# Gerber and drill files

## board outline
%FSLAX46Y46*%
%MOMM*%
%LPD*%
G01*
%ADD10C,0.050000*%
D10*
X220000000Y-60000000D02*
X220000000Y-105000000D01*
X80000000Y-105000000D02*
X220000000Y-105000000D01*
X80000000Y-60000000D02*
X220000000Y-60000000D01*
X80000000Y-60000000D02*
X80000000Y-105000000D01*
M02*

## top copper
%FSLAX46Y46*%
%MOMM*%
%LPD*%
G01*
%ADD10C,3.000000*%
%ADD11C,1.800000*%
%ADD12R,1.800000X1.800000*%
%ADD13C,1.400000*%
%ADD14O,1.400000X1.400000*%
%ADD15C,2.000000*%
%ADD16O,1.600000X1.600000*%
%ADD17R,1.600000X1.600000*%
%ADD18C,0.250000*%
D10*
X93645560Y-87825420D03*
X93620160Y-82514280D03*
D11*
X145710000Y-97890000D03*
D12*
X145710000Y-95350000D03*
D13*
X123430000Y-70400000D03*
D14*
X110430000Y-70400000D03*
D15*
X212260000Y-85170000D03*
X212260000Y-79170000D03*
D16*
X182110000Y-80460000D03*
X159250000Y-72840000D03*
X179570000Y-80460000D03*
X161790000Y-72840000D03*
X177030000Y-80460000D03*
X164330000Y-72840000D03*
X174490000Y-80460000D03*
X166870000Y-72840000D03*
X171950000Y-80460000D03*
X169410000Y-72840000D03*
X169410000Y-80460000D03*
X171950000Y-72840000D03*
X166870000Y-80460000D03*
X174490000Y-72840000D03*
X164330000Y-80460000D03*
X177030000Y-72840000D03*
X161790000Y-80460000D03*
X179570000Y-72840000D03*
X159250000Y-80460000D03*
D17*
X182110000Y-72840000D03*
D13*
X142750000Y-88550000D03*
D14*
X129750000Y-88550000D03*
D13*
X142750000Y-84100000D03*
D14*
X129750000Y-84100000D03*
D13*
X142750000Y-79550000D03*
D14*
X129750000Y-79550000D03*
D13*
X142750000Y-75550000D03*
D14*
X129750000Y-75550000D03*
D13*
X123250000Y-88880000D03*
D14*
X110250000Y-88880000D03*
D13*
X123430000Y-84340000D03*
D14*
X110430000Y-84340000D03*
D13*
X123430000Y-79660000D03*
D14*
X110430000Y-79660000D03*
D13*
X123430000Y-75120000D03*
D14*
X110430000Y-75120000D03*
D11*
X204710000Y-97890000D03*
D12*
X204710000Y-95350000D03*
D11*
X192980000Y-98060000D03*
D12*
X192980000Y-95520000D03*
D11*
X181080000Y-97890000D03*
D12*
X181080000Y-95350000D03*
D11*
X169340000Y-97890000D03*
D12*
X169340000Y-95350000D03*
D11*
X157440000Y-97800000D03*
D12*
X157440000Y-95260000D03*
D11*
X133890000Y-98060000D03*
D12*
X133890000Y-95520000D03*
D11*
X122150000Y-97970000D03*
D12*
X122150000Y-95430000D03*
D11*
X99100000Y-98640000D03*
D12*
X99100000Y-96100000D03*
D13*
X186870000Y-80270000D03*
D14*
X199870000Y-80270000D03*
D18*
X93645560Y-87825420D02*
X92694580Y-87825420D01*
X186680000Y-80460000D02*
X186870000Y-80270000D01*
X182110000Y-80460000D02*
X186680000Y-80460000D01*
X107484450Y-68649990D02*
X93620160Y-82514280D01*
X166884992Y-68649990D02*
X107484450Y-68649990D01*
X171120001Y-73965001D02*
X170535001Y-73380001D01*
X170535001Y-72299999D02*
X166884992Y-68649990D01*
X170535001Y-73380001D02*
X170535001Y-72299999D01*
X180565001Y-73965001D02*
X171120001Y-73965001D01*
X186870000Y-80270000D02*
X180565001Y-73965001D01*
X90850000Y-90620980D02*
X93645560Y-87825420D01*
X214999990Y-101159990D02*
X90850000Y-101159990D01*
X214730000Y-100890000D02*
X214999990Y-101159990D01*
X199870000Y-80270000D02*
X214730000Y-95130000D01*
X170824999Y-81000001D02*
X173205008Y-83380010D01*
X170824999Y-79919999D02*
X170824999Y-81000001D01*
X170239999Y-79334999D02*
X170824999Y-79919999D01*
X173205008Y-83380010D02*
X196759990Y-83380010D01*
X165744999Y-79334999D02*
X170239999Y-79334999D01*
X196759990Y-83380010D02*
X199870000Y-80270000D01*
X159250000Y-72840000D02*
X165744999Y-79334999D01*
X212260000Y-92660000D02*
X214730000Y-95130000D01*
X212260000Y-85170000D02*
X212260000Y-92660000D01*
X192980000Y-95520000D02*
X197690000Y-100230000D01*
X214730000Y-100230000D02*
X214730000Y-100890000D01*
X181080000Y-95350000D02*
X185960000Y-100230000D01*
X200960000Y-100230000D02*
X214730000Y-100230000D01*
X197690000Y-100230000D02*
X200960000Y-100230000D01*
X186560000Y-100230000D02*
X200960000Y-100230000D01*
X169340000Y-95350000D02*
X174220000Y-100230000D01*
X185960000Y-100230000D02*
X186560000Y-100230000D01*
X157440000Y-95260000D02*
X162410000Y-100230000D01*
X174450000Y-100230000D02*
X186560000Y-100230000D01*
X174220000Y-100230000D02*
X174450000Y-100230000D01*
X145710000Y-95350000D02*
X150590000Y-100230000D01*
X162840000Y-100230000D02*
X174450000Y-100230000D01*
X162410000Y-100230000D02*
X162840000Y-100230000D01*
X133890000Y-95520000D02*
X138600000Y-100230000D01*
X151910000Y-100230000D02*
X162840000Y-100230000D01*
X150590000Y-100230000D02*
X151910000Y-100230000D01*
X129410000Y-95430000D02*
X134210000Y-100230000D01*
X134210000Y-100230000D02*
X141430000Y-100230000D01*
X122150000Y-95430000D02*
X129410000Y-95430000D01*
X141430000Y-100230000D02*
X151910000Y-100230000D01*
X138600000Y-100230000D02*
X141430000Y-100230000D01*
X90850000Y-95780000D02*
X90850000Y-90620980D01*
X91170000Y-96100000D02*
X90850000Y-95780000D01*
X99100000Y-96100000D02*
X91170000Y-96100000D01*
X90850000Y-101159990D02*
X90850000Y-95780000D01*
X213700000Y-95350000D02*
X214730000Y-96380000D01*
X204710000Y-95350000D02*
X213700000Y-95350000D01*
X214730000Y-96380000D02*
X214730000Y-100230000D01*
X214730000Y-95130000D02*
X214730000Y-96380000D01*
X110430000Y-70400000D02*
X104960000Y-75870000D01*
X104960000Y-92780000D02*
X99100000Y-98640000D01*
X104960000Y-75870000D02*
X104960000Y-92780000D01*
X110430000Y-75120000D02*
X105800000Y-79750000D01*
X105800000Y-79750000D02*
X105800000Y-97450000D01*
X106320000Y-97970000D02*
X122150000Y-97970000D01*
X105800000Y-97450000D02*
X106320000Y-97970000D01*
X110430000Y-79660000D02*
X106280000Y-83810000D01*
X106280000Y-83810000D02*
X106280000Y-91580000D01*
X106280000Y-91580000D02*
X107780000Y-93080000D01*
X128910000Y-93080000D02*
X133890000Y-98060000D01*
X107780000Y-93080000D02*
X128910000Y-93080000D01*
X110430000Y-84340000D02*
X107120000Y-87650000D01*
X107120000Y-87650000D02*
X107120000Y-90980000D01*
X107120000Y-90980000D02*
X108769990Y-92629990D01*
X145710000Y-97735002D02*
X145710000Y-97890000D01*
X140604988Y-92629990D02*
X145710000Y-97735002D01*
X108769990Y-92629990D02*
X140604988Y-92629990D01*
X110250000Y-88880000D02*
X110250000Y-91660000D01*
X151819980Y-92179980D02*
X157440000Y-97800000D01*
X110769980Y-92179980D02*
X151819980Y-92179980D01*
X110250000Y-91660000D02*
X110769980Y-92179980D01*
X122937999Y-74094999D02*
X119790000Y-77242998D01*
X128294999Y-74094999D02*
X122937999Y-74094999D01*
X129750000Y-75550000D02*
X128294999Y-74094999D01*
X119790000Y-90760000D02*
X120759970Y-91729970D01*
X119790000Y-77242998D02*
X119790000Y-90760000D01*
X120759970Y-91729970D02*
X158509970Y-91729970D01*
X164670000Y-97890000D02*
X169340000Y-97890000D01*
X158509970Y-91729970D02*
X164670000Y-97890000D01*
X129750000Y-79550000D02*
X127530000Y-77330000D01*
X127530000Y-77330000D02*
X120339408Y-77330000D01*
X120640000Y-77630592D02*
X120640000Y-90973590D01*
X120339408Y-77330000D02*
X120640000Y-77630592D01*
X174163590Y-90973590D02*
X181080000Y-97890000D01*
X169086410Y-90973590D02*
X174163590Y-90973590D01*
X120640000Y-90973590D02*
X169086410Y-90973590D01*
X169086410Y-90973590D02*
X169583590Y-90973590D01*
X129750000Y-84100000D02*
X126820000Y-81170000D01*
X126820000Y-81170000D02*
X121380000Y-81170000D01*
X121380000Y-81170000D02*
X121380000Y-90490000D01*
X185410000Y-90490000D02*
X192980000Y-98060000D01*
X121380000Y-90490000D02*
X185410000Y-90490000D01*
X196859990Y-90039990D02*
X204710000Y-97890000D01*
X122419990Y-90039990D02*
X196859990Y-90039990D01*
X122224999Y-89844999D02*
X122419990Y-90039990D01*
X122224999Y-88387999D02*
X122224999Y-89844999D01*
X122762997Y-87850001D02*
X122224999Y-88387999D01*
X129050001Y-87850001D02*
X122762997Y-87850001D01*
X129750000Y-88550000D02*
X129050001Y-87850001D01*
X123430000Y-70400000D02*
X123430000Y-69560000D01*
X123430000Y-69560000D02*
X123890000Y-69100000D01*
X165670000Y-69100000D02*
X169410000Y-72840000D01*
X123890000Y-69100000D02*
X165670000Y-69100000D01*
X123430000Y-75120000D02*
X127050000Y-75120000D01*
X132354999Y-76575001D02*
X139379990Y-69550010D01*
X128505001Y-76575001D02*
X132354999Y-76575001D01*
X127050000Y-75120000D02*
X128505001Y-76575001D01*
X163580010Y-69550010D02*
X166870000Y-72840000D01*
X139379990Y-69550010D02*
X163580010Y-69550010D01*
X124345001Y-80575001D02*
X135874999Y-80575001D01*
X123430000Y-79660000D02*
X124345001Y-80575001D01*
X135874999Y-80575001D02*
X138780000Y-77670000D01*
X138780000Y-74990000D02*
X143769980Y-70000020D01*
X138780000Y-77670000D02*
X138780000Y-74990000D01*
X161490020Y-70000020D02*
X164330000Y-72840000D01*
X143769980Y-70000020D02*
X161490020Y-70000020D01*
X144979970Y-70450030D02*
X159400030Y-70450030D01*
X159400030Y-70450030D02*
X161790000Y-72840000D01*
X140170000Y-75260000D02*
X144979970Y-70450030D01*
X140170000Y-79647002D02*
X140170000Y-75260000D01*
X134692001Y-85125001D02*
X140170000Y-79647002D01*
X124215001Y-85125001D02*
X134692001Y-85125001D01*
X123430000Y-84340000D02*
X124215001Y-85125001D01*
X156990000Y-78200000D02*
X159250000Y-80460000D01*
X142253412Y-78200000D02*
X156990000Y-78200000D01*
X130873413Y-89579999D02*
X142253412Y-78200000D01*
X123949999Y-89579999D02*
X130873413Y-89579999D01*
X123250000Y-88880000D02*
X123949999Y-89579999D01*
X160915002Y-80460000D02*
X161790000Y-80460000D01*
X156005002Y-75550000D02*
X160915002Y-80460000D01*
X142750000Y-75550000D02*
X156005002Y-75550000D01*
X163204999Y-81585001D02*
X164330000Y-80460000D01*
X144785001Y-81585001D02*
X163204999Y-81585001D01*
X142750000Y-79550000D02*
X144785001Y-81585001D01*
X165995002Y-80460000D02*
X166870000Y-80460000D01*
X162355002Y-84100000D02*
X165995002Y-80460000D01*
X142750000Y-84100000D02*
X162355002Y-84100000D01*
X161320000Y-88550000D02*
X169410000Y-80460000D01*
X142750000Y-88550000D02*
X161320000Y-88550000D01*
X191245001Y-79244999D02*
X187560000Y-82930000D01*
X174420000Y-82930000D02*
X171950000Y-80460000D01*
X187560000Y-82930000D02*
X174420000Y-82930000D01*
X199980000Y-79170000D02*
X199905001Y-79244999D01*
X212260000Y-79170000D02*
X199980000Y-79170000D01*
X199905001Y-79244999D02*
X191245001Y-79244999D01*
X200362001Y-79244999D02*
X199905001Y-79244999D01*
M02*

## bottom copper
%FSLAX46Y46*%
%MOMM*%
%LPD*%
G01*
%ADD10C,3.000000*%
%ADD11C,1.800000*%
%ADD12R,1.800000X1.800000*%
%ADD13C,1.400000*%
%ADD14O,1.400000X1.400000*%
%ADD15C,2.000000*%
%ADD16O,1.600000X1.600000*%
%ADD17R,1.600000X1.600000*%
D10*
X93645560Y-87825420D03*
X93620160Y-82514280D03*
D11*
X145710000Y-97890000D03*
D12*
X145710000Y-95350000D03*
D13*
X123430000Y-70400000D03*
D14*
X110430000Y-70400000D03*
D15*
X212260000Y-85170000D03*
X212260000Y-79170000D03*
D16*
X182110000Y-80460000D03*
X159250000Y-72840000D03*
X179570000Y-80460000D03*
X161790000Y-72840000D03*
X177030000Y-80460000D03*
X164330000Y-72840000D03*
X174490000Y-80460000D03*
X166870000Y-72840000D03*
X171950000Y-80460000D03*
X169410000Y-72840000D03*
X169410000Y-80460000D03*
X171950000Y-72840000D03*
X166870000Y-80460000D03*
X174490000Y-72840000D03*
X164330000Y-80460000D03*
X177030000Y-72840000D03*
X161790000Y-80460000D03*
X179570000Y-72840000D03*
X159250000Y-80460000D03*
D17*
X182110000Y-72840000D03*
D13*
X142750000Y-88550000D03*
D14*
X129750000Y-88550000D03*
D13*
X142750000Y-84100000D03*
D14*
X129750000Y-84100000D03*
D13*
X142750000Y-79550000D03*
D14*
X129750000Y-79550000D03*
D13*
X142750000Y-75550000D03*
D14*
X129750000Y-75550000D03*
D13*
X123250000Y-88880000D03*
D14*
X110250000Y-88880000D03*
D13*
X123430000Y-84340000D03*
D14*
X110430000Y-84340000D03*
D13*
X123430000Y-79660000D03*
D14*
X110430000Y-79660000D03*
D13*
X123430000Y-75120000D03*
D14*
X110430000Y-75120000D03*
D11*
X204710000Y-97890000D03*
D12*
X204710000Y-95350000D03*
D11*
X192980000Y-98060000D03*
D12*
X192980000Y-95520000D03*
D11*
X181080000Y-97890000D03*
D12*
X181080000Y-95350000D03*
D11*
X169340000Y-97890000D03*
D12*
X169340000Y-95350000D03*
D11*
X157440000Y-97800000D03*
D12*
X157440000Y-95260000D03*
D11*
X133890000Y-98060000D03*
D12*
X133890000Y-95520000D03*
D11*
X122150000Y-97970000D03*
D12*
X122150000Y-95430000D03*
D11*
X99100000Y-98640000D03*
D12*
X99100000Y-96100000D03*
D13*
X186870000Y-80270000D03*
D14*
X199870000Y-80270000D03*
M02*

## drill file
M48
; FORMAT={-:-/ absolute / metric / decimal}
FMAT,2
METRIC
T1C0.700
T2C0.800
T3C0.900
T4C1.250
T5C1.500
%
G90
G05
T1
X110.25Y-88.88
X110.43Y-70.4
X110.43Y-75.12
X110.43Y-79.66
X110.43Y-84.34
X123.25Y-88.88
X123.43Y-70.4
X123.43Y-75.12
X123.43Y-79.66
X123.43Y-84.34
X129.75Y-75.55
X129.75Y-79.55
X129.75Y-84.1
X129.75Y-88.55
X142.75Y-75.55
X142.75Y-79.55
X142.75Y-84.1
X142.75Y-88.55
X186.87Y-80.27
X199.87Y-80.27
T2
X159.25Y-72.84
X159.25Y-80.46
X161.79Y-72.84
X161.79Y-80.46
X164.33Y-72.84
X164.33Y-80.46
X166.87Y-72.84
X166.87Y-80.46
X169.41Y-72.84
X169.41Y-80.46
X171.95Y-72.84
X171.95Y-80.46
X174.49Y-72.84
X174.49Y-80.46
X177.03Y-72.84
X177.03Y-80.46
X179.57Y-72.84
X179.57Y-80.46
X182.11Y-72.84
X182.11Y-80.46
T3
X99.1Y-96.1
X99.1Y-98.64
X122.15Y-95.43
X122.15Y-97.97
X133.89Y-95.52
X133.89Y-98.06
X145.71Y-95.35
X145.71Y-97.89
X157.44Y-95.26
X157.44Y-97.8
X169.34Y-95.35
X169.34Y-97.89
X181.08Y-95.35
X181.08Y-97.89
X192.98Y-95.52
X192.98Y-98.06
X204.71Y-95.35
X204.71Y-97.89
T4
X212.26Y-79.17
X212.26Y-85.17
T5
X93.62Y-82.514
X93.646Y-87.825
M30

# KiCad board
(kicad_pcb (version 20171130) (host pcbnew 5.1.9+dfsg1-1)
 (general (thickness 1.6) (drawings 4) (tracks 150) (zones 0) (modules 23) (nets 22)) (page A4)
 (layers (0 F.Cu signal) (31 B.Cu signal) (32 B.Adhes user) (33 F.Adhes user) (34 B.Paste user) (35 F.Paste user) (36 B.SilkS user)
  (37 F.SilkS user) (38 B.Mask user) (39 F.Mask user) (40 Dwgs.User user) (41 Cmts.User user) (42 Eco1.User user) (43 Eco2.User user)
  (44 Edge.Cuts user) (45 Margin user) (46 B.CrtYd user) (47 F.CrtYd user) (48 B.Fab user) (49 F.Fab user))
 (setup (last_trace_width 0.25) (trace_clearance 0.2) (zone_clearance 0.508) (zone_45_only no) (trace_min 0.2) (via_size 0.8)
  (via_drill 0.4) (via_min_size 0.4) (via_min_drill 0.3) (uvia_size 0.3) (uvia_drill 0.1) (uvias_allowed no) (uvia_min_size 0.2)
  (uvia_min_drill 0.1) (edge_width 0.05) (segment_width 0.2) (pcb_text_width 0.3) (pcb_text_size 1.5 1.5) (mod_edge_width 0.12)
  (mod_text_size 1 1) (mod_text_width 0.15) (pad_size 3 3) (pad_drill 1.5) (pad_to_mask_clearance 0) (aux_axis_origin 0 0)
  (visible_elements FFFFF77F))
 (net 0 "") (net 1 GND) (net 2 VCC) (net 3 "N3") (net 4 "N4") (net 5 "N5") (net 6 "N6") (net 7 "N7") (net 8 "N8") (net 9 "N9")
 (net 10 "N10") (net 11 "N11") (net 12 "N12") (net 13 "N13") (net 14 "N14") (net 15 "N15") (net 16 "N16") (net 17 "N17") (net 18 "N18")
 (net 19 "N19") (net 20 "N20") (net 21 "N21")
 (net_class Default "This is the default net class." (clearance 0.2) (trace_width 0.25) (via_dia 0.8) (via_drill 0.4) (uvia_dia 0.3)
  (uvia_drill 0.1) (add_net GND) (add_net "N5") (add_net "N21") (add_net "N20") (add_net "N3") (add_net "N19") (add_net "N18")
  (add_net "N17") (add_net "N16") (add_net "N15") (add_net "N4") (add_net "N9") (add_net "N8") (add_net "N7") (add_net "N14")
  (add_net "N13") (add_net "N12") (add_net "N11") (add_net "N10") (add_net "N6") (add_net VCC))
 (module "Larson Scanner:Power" (layer F.Cu) (at 93.61 85.1)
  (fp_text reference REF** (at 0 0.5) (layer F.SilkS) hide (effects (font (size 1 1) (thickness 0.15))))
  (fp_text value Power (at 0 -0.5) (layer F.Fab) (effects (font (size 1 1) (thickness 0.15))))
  (pad 2 thru_hole circle (at 0.03556 2.72542) (size 3 3) (drill 1.5) (layers *.Cu *.Mask) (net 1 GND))
  (pad 1 thru_hole circle (at 0.01016 -2.58572) (size 3 3) (drill 1.5) (layers *.Cu *.Mask) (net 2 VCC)))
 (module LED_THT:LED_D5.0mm (layer F.Cu) (at 145.71 95.35 270)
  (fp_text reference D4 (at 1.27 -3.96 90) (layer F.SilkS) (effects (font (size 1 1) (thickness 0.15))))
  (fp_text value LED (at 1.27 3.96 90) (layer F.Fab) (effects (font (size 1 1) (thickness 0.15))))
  (pad 2 thru_hole circle (at 2.54 0 270) (size 1.8 1.8) (drill 0.9) (layers *.Cu *.Mask) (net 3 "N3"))
  (pad 1 thru_hole rect (at 0 0 270) (size 1.8 1.8) (drill 0.9) (layers *.Cu *.Mask) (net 1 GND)))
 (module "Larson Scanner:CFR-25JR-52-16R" (layer F.Cu) (at 116.93 70.4 180)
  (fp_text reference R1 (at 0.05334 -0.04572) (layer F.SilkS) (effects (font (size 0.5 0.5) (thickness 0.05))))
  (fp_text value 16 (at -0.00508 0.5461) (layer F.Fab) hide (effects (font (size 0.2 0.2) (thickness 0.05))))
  (pad 1 thru_hole circle (at -6.5 0 180) (size 1.4 1.4) (drill 0.7) (layers *.Cu *.Mask) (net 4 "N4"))
  (pad 2 thru_hole oval (at 6.5 0 180) (size 1.4 1.4) (drill 0.7) (layers *.Cu *.Mask) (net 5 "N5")))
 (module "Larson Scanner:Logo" (layer F.Cu) (at 98.32 68.52)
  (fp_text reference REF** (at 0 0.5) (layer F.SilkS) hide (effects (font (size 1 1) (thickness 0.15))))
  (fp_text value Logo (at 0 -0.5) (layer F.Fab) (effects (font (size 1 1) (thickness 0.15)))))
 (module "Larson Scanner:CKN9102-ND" (layer F.Cu) (at 212.26 82.17)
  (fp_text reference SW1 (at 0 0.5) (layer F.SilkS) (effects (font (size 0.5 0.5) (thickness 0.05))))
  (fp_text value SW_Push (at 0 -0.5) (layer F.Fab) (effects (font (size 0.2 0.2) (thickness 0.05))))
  (pad 2 thru_hole circle (at 0 3 180) (size 2 2) (drill 1.25) (layers *.Cu *.Mask) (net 1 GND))
  (pad 1 thru_hole circle (at 0 -3 180) (size 2 2) (drill 1.25) (layers *.Cu *.Mask) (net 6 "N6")))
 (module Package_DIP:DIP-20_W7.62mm (layer F.Cu) (at 182.11 72.84 270)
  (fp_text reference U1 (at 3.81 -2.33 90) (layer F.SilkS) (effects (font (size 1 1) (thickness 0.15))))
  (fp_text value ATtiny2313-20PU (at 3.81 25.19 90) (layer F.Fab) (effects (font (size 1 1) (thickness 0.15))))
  (pad 20 thru_hole oval (at 7.62 0 270) (size 1.6 1.6) (drill 0.8) (layers *.Cu *.Mask) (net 2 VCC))
  (pad 10 thru_hole oval (at 0 22.86 270) (size 1.6 1.6) (drill 0.8) (layers *.Cu *.Mask) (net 1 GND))
  (pad 19 thru_hole oval (at 7.62 2.54 270) (size 1.6 1.6) (drill 0.8) (layers *.Cu *.Mask))
  (pad 9 thru_hole oval (at 0 20.32 270) (size 1.6 1.6) (drill 0.8) (layers *.Cu *.Mask) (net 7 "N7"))
  (pad 18 thru_hole oval (at 7.62 5.08 270) (size 1.6 1.6) (drill 0.8) (layers *.Cu *.Mask))
  (pad 8 thru_hole oval (at 0 17.78 270) (size 1.6 1.6) (drill 0.8) (layers *.Cu *.Mask) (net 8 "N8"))
  (pad 17 thru_hole oval (at 7.62 7.62 270) (size 1.6 1.6) (drill 0.8) (layers *.Cu *.Mask))
  (pad 7 thru_hole oval (at 0 15.24 270) (size 1.6 1.6) (drill 0.8) (layers *.Cu *.Mask) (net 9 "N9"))
  (pad 16 thru_hole oval (at 7.62 10.16 270) (size 1.6 1.6) (drill 0.8) (layers *.Cu *.Mask) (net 6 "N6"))
  (pad 6 thru_hole oval (at 0 12.7 270) (size 1.6 1.6) (drill 0.8) (layers *.Cu *.Mask) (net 4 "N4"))
  (pad 15 thru_hole oval (at 7.62 12.7 270) (size 1.6 1.6) (drill 0.8) (layers *.Cu *.Mask) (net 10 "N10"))
  (pad 5 thru_hole oval (at 0 10.16 270) (size 1.6 1.6) (drill 0.8) (layers *.Cu *.Mask))
  (pad 14 thru_hole oval (at 7.62 15.24 270) (size 1.6 1.6) (drill 0.8) (layers *.Cu *.Mask) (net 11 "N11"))
  (pad 4 thru_hole oval (at 0 7.62 270) (size 1.6 1.6) (drill 0.8) (layers *.Cu *.Mask))
  (pad 13 thru_hole oval (at 7.62 17.78 270) (size 1.6 1.6) (drill 0.8) (layers *.Cu *.Mask) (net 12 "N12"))
  (pad 3 thru_hole oval (at 0 5.08 270) (size 1.6 1.6) (drill 0.8) (layers *.Cu *.Mask))
  (pad 12 thru_hole oval (at 7.62 20.32 270) (size 1.6 1.6) (drill 0.8) (layers *.Cu *.Mask) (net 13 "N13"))
  (pad 2 thru_hole oval (at 0 2.54 270) (size 1.6 1.6) (drill 0.8) (layers *.Cu *.Mask))
  (pad 11 thru_hole oval (at 7.62 22.86 270) (size 1.6 1.6) (drill 0.8) (layers *.Cu *.Mask) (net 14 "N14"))
  (pad 1 thru_hole rect (at 0 0 270) (size 1.6 1.6) (drill 0.8) (layers *.Cu *.Mask)))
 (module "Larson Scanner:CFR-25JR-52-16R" (layer F.Cu) (at 136.25 88.55 180)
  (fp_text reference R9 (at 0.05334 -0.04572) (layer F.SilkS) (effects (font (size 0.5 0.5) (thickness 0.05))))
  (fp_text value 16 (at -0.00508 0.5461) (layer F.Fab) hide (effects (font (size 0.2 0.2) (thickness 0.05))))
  (pad 1 thru_hole circle (at -6.5 0 180) (size 1.4 1.4) (drill 0.7) (layers *.Cu *.Mask) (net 10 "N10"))
  (pad 2 thru_hole oval (at 6.5 0 180) (size 1.4 1.4) (drill 0.7) (layers *.Cu *.Mask) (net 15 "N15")))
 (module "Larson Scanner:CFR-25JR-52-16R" (layer F.Cu) (at 136.25 84.1 180)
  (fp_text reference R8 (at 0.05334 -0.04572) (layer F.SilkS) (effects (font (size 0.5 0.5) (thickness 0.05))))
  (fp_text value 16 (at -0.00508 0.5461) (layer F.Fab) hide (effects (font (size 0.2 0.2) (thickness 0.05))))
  (pad 1 thru_hole circle (at -6.5 0 180) (size 1.4 1.4) (drill 0.7) (layers *.Cu *.Mask) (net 11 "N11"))
  (pad 2 thru_hole oval (at 6.5 0 180) (size 1.4 1.4) (drill 0.7) (layers *.Cu *.Mask) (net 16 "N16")))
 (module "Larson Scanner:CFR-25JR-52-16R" (layer F.Cu) (at 136.25 79.55 180)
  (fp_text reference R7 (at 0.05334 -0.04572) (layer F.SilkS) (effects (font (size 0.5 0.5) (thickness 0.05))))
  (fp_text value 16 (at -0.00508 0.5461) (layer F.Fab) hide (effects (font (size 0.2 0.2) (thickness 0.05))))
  (pad 1 thru_hole circle (at -6.5 0 180) (size 1.4 1.4) (drill 0.7) (layers *.Cu *.Mask) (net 12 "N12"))
  (pad 2 thru_hole oval (at 6.5 0 180) (size 1.4 1.4) (drill 0.7) (layers *.Cu *.Mask) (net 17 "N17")))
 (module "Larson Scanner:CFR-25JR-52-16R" (layer F.Cu) (at 136.25 75.55 180)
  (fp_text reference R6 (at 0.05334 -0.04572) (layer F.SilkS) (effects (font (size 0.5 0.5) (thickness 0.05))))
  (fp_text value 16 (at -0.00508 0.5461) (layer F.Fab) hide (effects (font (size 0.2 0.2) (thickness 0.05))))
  (pad 1 thru_hole circle (at -6.5 0 180) (size 1.4 1.4) (drill 0.7) (layers *.Cu *.Mask) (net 13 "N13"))
  (pad 2 thru_hole oval (at 6.5 0 180) (size 1.4 1.4) (drill 0.7) (layers *.Cu *.Mask) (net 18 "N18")))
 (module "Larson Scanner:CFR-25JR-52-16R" (layer F.Cu) (at 116.75 88.88 180)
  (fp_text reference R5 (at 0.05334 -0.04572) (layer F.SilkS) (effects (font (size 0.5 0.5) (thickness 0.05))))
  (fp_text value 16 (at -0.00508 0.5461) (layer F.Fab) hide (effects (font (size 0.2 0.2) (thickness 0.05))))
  (pad 1 thru_hole circle (at -6.5 0 180) (size 1.4 1.4) (drill 0.7) (layers *.Cu *.Mask) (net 14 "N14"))
  (pad 2 thru_hole oval (at 6.5 0 180) (size 1.4 1.4) (drill 0.7) (layers *.Cu *.Mask) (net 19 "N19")))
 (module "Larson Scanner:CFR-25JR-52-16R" (layer F.Cu) (at 116.93 84.34 180)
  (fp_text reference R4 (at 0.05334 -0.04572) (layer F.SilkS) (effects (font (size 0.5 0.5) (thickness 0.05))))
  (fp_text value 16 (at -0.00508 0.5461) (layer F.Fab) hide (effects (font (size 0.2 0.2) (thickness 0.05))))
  (pad 1 thru_hole circle (at -6.5 0 180) (size 1.4 1.4) (drill 0.7) (layers *.Cu *.Mask) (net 7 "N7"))
  (pad 2 thru_hole oval (at 6.5 0 180) (size 1.4 1.4) (drill 0.7) (layers *.Cu *.Mask) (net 3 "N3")))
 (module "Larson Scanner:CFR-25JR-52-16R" (layer F.Cu) (at 116.93 79.66 180)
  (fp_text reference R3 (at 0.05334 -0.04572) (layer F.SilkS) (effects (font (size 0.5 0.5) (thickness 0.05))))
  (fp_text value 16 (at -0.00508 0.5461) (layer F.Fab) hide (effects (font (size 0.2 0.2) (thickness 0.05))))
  (pad 1 thru_hole circle (at -6.5 0 180) (size 1.4 1.4) (drill 0.7) (layers *.Cu *.Mask) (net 8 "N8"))
  (pad 2 thru_hole oval (at 6.5 0 180) (size 1.4 1.4) (drill 0.7) (layers *.Cu *.Mask) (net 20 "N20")))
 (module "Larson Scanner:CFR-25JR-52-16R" (layer F.Cu) (at 116.93 75.12 180)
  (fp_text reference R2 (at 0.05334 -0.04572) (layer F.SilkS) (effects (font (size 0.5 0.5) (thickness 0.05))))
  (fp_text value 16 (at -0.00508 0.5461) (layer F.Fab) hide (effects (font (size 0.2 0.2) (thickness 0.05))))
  (pad 1 thru_hole circle (at -6.5 0 180) (size 1.4 1.4) (drill 0.7) (layers *.Cu *.Mask) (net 9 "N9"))
  (pad 2 thru_hole oval (at 6.5 0 180) (size 1.4 1.4) (drill 0.7) (layers *.Cu *.Mask) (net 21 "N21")))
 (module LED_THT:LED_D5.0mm (layer F.Cu) (at 204.71 95.35 270)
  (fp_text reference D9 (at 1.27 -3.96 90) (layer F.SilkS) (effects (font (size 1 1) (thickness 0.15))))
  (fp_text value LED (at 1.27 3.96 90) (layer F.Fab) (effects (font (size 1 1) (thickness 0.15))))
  (pad 2 thru_hole circle (at 2.54 0 270) (size 1.8 1.8) (drill 0.9) (layers *.Cu *.Mask) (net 15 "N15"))
  (pad 1 thru_hole rect (at 0 0 270) (size 1.8 1.8) (drill 0.9) (layers *.Cu *.Mask) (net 1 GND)))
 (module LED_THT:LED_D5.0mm (layer F.Cu) (at 192.98 95.52 270)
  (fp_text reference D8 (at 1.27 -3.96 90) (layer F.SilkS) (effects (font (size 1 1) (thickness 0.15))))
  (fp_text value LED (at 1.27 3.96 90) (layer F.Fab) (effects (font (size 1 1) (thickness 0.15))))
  (pad 2 thru_hole circle (at 2.54 0 270) (size 1.8 1.8) (drill 0.9) (layers *.Cu *.Mask) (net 16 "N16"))
  (pad 1 thru_hole rect (at 0 0 270) (size 1.8 1.8) (drill 0.9) (layers *.Cu *.Mask) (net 1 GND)))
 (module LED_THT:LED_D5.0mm (layer F.Cu) (at 181.08 95.35 270)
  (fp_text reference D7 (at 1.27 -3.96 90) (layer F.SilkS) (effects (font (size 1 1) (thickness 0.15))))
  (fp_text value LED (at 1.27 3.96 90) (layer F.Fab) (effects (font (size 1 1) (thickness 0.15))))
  (pad 2 thru_hole circle (at 2.54 0 270) (size 1.8 1.8) (drill 0.9) (layers *.Cu *.Mask) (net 17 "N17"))
  (pad 1 thru_hole rect (at 0 0 270) (size 1.8 1.8) (drill 0.9) (layers *.Cu *.Mask) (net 1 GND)))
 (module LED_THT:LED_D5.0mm (layer F.Cu) (at 169.34 95.35 270)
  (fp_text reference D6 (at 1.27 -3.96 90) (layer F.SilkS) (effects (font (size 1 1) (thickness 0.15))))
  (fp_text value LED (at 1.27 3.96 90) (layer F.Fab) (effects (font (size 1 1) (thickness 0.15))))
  (pad 2 thru_hole circle (at 2.54 0 270) (size 1.8 1.8) (drill 0.9) (layers *.Cu *.Mask) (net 18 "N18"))
  (pad 1 thru_hole rect (at 0 0 270) (size 1.8 1.8) (drill 0.9) (layers *.Cu *.Mask) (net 1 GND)))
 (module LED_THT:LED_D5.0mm (layer F.Cu) (at 157.44 95.26 270)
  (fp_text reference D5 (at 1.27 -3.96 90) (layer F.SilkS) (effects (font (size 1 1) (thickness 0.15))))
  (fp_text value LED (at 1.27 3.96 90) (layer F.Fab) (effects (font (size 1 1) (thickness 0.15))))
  (pad 2 thru_hole circle (at 2.54 0 270) (size 1.8 1.8) (drill 0.9) (layers *.Cu *.Mask) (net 19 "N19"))
  (pad 1 thru_hole rect (at 0 0 270) (size 1.8 1.8) (drill 0.9) (layers *.Cu *.Mask) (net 1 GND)))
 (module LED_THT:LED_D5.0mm (layer F.Cu) (at 133.89 95.52 270)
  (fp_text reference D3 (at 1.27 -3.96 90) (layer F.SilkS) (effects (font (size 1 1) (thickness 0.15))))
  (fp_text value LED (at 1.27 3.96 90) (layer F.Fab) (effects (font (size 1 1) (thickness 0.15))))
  (pad 2 thru_hole circle (at 2.54 0 270) (size 1.8 1.8) (drill 0.9) (layers *.Cu *.Mask) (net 20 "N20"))
  (pad 1 thru_hole rect (at 0 0 270) (size 1.8 1.8) (drill 0.9) (layers *.Cu *.Mask) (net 1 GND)))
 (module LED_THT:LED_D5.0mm (layer F.Cu) (at 122.15 95.43 270)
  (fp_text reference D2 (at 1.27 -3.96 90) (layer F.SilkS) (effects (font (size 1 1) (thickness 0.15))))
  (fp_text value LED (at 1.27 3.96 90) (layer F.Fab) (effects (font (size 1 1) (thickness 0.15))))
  (pad 2 thru_hole circle (at 2.54 0 270) (size 1.8 1.8) (drill 0.9) (layers *.Cu *.Mask) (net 21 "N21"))
  (pad 1 thru_hole rect (at 0 0 270) (size 1.8 1.8) (drill 0.9) (layers *.Cu *.Mask) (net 1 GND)))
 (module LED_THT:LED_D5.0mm (layer F.Cu) (at 99.1 96.1 270)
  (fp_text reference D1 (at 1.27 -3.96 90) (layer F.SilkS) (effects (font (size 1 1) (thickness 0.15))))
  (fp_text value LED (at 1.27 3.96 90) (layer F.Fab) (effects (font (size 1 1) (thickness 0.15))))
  (pad 2 thru_hole circle (at 2.54 0 270) (size 1.8 1.8) (drill 0.9) (layers *.Cu *.Mask) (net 5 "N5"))
  (pad 1 thru_hole rect (at 0 0 270) (size 1.8 1.8) (drill 0.9) (layers *.Cu *.Mask) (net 1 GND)))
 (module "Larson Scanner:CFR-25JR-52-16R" (layer F.Cu) (at 193.37 80.27)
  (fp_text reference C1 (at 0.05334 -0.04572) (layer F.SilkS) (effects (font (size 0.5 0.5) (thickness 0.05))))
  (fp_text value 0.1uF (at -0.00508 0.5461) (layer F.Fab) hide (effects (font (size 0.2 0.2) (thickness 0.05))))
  (pad 1 thru_hole circle (at -6.5 0) (size 1.4 1.4) (drill 0.7) (layers *.Cu *.Mask) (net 2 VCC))
  (pad 2 thru_hole oval (at 6.5 0) (size 1.4 1.4) (drill 0.7) (layers *.Cu *.Mask) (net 1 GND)))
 (gr_line (start 220 60) (end 220 105) (layer Edge.Cuts) (width 0.05))
 (gr_line (start 80 105) (end 220 105) (layer Edge.Cuts) (width 0.05))
 (gr_line (start 80 60) (end 220 60) (layer Edge.Cuts) (width 0.05))
 (gr_line (start 80 60) (end 80 105) (layer Edge.Cuts) (width 0.05))
 (segment (start 93.64556 87.82542) (end 92.69458 87.82542) (width 0.25) (layer F.Cu) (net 1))
 (segment (start 186.68 80.46) (end 186.87 80.27) (width 0.25) (layer F.Cu) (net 2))
 (segment (start 182.11 80.46) (end 186.68 80.46) (width 0.25) (layer F.Cu) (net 2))
 (segment (start 107.48445 68.64999) (end 93.62016 82.51428) (width 0.25) (layer F.Cu) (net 2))
 (segment (start 166.884992 68.64999) (end 107.48445 68.64999) (width 0.25) (layer F.Cu) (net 2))
 (segment (start 171.120001 73.965001) (end 170.535001 73.380001) (width 0.25) (layer F.Cu) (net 2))
 (segment (start 170.535001 72.299999) (end 166.884992 68.64999) (width 0.25) (layer F.Cu) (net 2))
 (segment (start 170.535001 73.380001) (end 170.535001 72.299999) (width 0.25) (layer F.Cu) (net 2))
 (segment (start 180.565001 73.965001) (end 171.120001 73.965001) (width 0.25) (layer F.Cu) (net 2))
 (segment (start 186.87 80.27) (end 180.565001 73.965001) (width 0.25) (layer F.Cu) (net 2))
 (segment (start 90.85 90.62098) (end 93.64556 87.82542) (width 0.25) (layer F.Cu) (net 1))
 (segment (start 214.99999 101.15999) (end 90.85 101.15999) (width 0.25) (layer F.Cu) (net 1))
 (segment (start 214.73 100.89) (end 214.99999 101.15999) (width 0.25) (layer F.Cu) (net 1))
 (segment (start 199.87 80.27) (end 214.73 95.13) (width 0.25) (layer F.Cu) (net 1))
 (segment (start 170.824999 81.000001) (end 173.205008 83.38001) (width 0.25) (layer F.Cu) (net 1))
 (segment (start 170.824999 79.919999) (end 170.824999 81.000001) (width 0.25) (layer F.Cu) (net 1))
 (segment (start 170.239999 79.334999) (end 170.824999 79.919999) (width 0.25) (layer F.Cu) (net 1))
 (segment (start 173.205008 83.38001) (end 196.75999 83.38001) (width 0.25) (layer F.Cu) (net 1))
 (segment (start 165.744999 79.334999) (end 170.239999 79.334999) (width 0.25) (layer F.Cu) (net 1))
 (segment (start 196.75999 83.38001) (end 199.87 80.27) (width 0.25) (layer F.Cu) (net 1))
 (segment (start 159.25 72.84) (end 165.744999 79.334999) (width 0.25) (layer F.Cu) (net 1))
 (segment (start 212.26 92.66) (end 214.73 95.13) (width 0.25) (layer F.Cu) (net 1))
 (segment (start 212.26 85.17) (end 212.26 92.66) (width 0.25) (layer F.Cu) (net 1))
 (segment (start 192.98 95.52) (end 197.69 100.23) (width 0.25) (layer F.Cu) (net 1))
 (segment (start 214.73 100.23) (end 214.73 100.89) (width 0.25) (layer F.Cu) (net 1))
 (segment (start 181.08 95.35) (end 185.96 100.23) (width 0.25) (layer F.Cu) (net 1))
 (segment (start 200.96 100.23) (end 214.73 100.23) (width 0.25) (layer F.Cu) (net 1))
 (segment (start 197.69 100.23) (end 200.96 100.23) (width 0.25) (layer F.Cu) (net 1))
 (segment (start 186.56 100.23) (end 200.96 100.23) (width 0.25) (layer F.Cu) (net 1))
 (segment (start 169.34 95.35) (end 174.22 100.23) (width 0.25) (layer F.Cu) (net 1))
 (segment (start 185.96 100.23) (end 186.56 100.23) (width 0.25) (layer F.Cu) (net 1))
 (segment (start 157.44 95.26) (end 162.41 100.23) (width 0.25) (layer F.Cu) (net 1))
 (segment (start 174.45 100.23) (end 186.56 100.23) (width 0.25) (layer F.Cu) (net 1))
 (segment (start 174.22 100.23) (end 174.45 100.23) (width 0.25) (layer F.Cu) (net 1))
 (segment (start 145.71 95.35) (end 150.59 100.23) (width 0.25) (layer F.Cu) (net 1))
 (segment (start 162.84 100.23) (end 174.45 100.23) (width 0.25) (layer F.Cu) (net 1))
 (segment (start 162.41 100.23) (end 162.84 100.23) (width 0.25) (layer F.Cu) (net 1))
 (segment (start 133.89 95.52) (end 138.6 100.23) (width 0.25) (layer F.Cu) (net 1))
 (segment (start 151.91 100.23) (end 162.84 100.23) (width 0.25) (layer F.Cu) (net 1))
 (segment (start 150.59 100.23) (end 151.91 100.23) (width 0.25) (layer F.Cu) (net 1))
 (segment (start 129.41 95.43) (end 134.21 100.23) (width 0.25) (layer F.Cu) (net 1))
 (segment (start 134.21 100.23) (end 141.43 100.23) (width 0.25) (layer F.Cu) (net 1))
 (segment (start 122.15 95.43) (end 129.41 95.43) (width 0.25) (layer F.Cu) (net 1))
 (segment (start 141.43 100.23) (end 151.91 100.23) (width 0.25) (layer F.Cu) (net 1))
 (segment (start 138.6 100.23) (end 141.43 100.23) (width 0.25) (layer F.Cu) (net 1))
 (segment (start 90.85 95.78) (end 90.85 90.62098) (width 0.25) (layer F.Cu) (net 1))
 (segment (start 91.17 96.1) (end 90.85 95.78) (width 0.25) (layer F.Cu) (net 1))
 (segment (start 99.1 96.1) (end 91.17 96.1) (width 0.25) (layer F.Cu) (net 1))
 (segment (start 90.85 101.15999) (end 90.85 95.78) (width 0.25) (layer F.Cu) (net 1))
 (segment (start 213.7 95.35) (end 214.73 96.38) (width 0.25) (layer F.Cu) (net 1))
 (segment (start 204.71 95.35) (end 213.7 95.35) (width 0.25) (layer F.Cu) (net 1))
 (segment (start 214.73 96.38) (end 214.73 100.23) (width 0.25) (layer F.Cu) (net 1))
 (segment (start 214.73 95.13) (end 214.73 96.38) (width 0.25) (layer F.Cu) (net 1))
 (segment (start 110.43 70.4) (end 104.96 75.87) (width 0.25) (layer F.Cu) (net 5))
 (segment (start 104.96 92.78) (end 99.1 98.64) (width 0.25) (layer F.Cu) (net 5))
 (segment (start 104.96 75.87) (end 104.96 92.78) (width 0.25) (layer F.Cu) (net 5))
 (segment (start 110.43 75.12) (end 105.8 79.75) (width 0.25) (layer F.Cu) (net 21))
 (segment (start 105.8 79.75) (end 105.8 97.45) (width 0.25) (layer F.Cu) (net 21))
 (segment (start 106.32 97.97) (end 122.15 97.97) (width 0.25) (layer F.Cu) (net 21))
 (segment (start 105.8 97.45) (end 106.32 97.97) (width 0.25) (layer F.Cu) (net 21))
 (segment (start 110.43 79.66) (end 106.28 83.81) (width 0.25) (layer F.Cu) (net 20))
 (segment (start 106.28 83.81) (end 106.28 91.58) (width 0.25) (layer F.Cu) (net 20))
 (segment (start 106.28 91.58) (end 107.78 93.08) (width 0.25) (layer F.Cu) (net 20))
 (segment (start 128.91 93.08) (end 133.89 98.06) (width 0.25) (layer F.Cu) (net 20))
 (segment (start 107.78 93.08) (end 128.91 93.08) (width 0.25) (layer F.Cu) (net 20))
 (segment (start 110.43 84.34) (end 107.12 87.65) (width 0.25) (layer F.Cu) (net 3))
 (segment (start 107.12 87.65) (end 107.12 90.98) (width 0.25) (layer F.Cu) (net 3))
 (segment (start 107.12 90.98) (end 108.76999 92.62999) (width 0.25) (layer F.Cu) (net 3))
 (segment (start 145.71 97.735002) (end 145.71 97.89) (width 0.25) (layer F.Cu) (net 3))
 (segment (start 140.604988 92.62999) (end 145.71 97.735002) (width 0.25) (layer F.Cu) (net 3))
 (segment (start 108.76999 92.62999) (end 140.604988 92.62999) (width 0.25) (layer F.Cu) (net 3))
 (segment (start 110.25 88.88) (end 110.25 91.66) (width 0.25) (layer F.Cu) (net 19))
 (segment (start 151.81998 92.17998) (end 157.44 97.8) (width 0.25) (layer F.Cu) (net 19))
 (segment (start 110.76998 92.17998) (end 151.81998 92.17998) (width 0.25) (layer F.Cu) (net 19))
 (segment (start 110.25 91.66) (end 110.76998 92.17998) (width 0.25) (layer F.Cu) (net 19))
 (segment (start 122.937999 74.094999) (end 119.79 77.242998) (width 0.25) (layer F.Cu) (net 18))
 (segment (start 128.294999 74.094999) (end 122.937999 74.094999) (width 0.25) (layer F.Cu) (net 18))
 (segment (start 129.75 75.55) (end 128.294999 74.094999) (width 0.25) (layer F.Cu) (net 18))
 (segment (start 119.79 90.76) (end 120.75997 91.72997) (width 0.25) (layer F.Cu) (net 18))
 (segment (start 119.79 77.242998) (end 119.79 90.76) (width 0.25) (layer F.Cu) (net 18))
 (segment (start 120.75997 91.72997) (end 158.50997 91.72997) (width 0.25) (layer F.Cu) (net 18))
 (segment (start 164.67 97.89) (end 169.34 97.89) (width 0.25) (layer F.Cu) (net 18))
 (segment (start 158.50997 91.72997) (end 164.67 97.89) (width 0.25) (layer F.Cu) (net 18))
 (segment (start 129.75 79.55) (end 127.53 77.33) (width 0.25) (layer F.Cu) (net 17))
 (segment (start 127.53 77.33) (end 120.339408 77.33) (width 0.25) (layer F.Cu) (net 17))
 (segment (start 120.64 77.630592) (end 120.64 90.97359) (width 0.25) (layer F.Cu) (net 17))
 (segment (start 120.339408 77.33) (end 120.64 77.630592) (width 0.25) (layer F.Cu) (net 17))
 (segment (start 174.16359 90.97359) (end 181.08 97.89) (width 0.25) (layer F.Cu) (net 17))
 (segment (start 169.08641 90.97359) (end 174.16359 90.97359) (width 0.25) (layer F.Cu) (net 17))
 (segment (start 120.64 90.97359) (end 169.08641 90.97359) (width 0.25) (layer F.Cu) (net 17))
 (segment (start 169.08641 90.97359) (end 169.58359 90.97359) (width 0.25) (layer F.Cu) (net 17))
 (segment (start 129.75 84.1) (end 126.82 81.17) (width 0.25) (layer F.Cu) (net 16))
 (segment (start 126.82 81.17) (end 121.38 81.17) (width 0.25) (layer F.Cu) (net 16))
 (segment (start 121.38 81.17) (end 121.38 90.49) (width 0.25) (layer F.Cu) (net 16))
 (segment (start 185.41 90.49) (end 192.98 98.06) (width 0.25) (layer F.Cu) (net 16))
 (segment (start 121.38 90.49) (end 185.41 90.49) (width 0.25) (layer F.Cu) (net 16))
 (segment (start 196.85999 90.03999) (end 204.71 97.89) (width 0.25) (layer F.Cu) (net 15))
 (segment (start 122.41999 90.03999) (end 196.85999 90.03999) (width 0.25) (layer F.Cu) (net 15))
 (segment (start 122.224999 89.844999) (end 122.41999 90.03999) (width 0.25) (layer F.Cu) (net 15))
 (segment (start 122.224999 88.387999) (end 122.224999 89.844999) (width 0.25) (layer F.Cu) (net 15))
 (segment (start 122.762997 87.850001) (end 122.224999 88.387999) (width 0.25) (layer F.Cu) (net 15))
 (segment (start 129.050001 87.850001) (end 122.762997 87.850001) (width 0.25) (layer F.Cu) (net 15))
 (segment (start 129.75 88.55) (end 129.050001 87.850001) (width 0.25) (layer F.Cu) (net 15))
 (segment (start 123.43 70.4) (end 123.43 69.56) (width 0.25) (layer F.Cu) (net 4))
 (segment (start 123.43 69.56) (end 123.89 69.1) (width 0.25) (layer F.Cu) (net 4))
 (segment (start 165.67 69.1) (end 169.41 72.84) (width 0.25) (layer F.Cu) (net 4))
 (segment (start 123.89 69.1) (end 165.67 69.1) (width 0.25) (layer F.Cu) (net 4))
 (segment (start 123.43 75.12) (end 127.05 75.12) (width 0.25) (layer F.Cu) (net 9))
 (segment (start 132.354999 76.575001) (end 139.37999 69.55001) (width 0.25) (layer F.Cu) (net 9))
 (segment (start 128.505001 76.575001) (end 132.354999 76.575001) (width 0.25) (layer F.Cu) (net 9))
 (segment (start 127.05 75.12) (end 128.505001 76.575001) (width 0.25) (layer F.Cu) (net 9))
 (segment (start 163.58001 69.55001) (end 166.87 72.84) (width 0.25) (layer F.Cu) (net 9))
 (segment (start 139.37999 69.55001) (end 163.58001 69.55001) (width 0.25) (layer F.Cu) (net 9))
 (segment (start 124.345001 80.575001) (end 135.874999 80.575001) (width 0.25) (layer F.Cu) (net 8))
 (segment (start 123.43 79.66) (end 124.345001 80.575001) (width 0.25) (layer F.Cu) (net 8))
 (segment (start 135.874999 80.575001) (end 138.78 77.67) (width 0.25) (layer F.Cu) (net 8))
 (segment (start 138.78 74.99) (end 143.76998 70.00002) (width 0.25) (layer F.Cu) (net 8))
 (segment (start 138.78 77.67) (end 138.78 74.99) (width 0.25) (layer F.Cu) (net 8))
 (segment (start 161.49002 70.00002) (end 164.33 72.84) (width 0.25) (layer F.Cu) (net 8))
 (segment (start 143.76998 70.00002) (end 161.49002 70.00002) (width 0.25) (layer F.Cu) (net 8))
 (segment (start 144.97997 70.45003) (end 159.40003 70.45003) (width 0.25) (layer F.Cu) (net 7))
 (segment (start 159.40003 70.45003) (end 161.79 72.84) (width 0.25) (layer F.Cu) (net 7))
 (segment (start 140.17 75.26) (end 144.97997 70.45003) (width 0.25) (layer F.Cu) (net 7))
 (segment (start 140.17 79.647002) (end 140.17 75.26) (width 0.25) (layer F.Cu) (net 7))
 (segment (start 134.692001 85.125001) (end 140.17 79.647002) (width 0.25) (layer F.Cu) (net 7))
 (segment (start 124.215001 85.125001) (end 134.692001 85.125001) (width 0.25) (layer F.Cu) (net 7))
 (segment (start 123.43 84.34) (end 124.215001 85.125001) (width 0.25) (layer F.Cu) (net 7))
 (segment (start 156.99 78.2) (end 159.25 80.46) (width 0.25) (layer F.Cu) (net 14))
 (segment (start 142.253412 78.2) (end 156.99 78.2) (width 0.25) (layer F.Cu) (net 14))
 (segment (start 130.873413 89.579999) (end 142.253412 78.2) (width 0.25) (layer F.Cu) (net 14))
 (segment (start 123.949999 89.579999) (end 130.873413 89.579999) (width 0.25) (layer F.Cu) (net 14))
 (segment (start 123.25 88.88) (end 123.949999 89.579999) (width 0.25) (layer F.Cu) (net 14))
 (segment (start 160.915002 80.46) (end 161.79 80.46) (width 0.25) (layer F.Cu) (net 13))
 (segment (start 156.005002 75.55) (end 160.915002 80.46) (width 0.25) (layer F.Cu) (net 13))
 (segment (start 142.75 75.55) (end 156.005002 75.55) (width 0.25) (layer F.Cu) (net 13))
 (segment (start 163.204999 81.585001) (end 164.33 80.46) (width 0.25) (layer F.Cu) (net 12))
 (segment (start 144.785001 81.585001) (end 163.204999 81.585001) (width 0.25) (layer F.Cu) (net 12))
 (segment (start 142.75 79.55) (end 144.785001 81.585001) (width 0.25) (layer F.Cu) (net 12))
 (segment (start 165.995002 80.46) (end 166.87 80.46) (width 0.25) (layer F.Cu) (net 11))
 (segment (start 162.355002 84.1) (end 165.995002 80.46) (width 0.25) (layer F.Cu) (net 11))
 (segment (start 142.75 84.1) (end 162.355002 84.1) (width 0.25) (layer F.Cu) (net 11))
 (segment (start 161.32 88.55) (end 169.41 80.46) (width 0.25) (layer F.Cu) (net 10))
 (segment (start 142.75 88.55) (end 161.32 88.55) (width 0.25) (layer F.Cu) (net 10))
 (segment (start 191.245001 79.244999) (end 187.56 82.93) (width 0.25) (layer F.Cu) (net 6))
 (segment (start 174.42 82.93) (end 171.95 80.46) (width 0.25) (layer F.Cu) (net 6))
 (segment (start 187.56 82.93) (end 174.42 82.93) (width 0.25) (layer F.Cu) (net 6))
 (segment (start 199.98 79.17) (end 199.905001 79.244999) (width 0.25) (layer F.Cu) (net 6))
 (segment (start 212.26 79.17) (end 199.98 79.17) (width 0.25) (layer F.Cu) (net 6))
 (segment (start 199.905001 79.244999) (end 191.245001 79.244999) (width 0.25) (layer F.Cu) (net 6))
 (segment (start 200.362001 79.244999) (end 199.905001 79.244999) (width 0.25) (layer F.Cu) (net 6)))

